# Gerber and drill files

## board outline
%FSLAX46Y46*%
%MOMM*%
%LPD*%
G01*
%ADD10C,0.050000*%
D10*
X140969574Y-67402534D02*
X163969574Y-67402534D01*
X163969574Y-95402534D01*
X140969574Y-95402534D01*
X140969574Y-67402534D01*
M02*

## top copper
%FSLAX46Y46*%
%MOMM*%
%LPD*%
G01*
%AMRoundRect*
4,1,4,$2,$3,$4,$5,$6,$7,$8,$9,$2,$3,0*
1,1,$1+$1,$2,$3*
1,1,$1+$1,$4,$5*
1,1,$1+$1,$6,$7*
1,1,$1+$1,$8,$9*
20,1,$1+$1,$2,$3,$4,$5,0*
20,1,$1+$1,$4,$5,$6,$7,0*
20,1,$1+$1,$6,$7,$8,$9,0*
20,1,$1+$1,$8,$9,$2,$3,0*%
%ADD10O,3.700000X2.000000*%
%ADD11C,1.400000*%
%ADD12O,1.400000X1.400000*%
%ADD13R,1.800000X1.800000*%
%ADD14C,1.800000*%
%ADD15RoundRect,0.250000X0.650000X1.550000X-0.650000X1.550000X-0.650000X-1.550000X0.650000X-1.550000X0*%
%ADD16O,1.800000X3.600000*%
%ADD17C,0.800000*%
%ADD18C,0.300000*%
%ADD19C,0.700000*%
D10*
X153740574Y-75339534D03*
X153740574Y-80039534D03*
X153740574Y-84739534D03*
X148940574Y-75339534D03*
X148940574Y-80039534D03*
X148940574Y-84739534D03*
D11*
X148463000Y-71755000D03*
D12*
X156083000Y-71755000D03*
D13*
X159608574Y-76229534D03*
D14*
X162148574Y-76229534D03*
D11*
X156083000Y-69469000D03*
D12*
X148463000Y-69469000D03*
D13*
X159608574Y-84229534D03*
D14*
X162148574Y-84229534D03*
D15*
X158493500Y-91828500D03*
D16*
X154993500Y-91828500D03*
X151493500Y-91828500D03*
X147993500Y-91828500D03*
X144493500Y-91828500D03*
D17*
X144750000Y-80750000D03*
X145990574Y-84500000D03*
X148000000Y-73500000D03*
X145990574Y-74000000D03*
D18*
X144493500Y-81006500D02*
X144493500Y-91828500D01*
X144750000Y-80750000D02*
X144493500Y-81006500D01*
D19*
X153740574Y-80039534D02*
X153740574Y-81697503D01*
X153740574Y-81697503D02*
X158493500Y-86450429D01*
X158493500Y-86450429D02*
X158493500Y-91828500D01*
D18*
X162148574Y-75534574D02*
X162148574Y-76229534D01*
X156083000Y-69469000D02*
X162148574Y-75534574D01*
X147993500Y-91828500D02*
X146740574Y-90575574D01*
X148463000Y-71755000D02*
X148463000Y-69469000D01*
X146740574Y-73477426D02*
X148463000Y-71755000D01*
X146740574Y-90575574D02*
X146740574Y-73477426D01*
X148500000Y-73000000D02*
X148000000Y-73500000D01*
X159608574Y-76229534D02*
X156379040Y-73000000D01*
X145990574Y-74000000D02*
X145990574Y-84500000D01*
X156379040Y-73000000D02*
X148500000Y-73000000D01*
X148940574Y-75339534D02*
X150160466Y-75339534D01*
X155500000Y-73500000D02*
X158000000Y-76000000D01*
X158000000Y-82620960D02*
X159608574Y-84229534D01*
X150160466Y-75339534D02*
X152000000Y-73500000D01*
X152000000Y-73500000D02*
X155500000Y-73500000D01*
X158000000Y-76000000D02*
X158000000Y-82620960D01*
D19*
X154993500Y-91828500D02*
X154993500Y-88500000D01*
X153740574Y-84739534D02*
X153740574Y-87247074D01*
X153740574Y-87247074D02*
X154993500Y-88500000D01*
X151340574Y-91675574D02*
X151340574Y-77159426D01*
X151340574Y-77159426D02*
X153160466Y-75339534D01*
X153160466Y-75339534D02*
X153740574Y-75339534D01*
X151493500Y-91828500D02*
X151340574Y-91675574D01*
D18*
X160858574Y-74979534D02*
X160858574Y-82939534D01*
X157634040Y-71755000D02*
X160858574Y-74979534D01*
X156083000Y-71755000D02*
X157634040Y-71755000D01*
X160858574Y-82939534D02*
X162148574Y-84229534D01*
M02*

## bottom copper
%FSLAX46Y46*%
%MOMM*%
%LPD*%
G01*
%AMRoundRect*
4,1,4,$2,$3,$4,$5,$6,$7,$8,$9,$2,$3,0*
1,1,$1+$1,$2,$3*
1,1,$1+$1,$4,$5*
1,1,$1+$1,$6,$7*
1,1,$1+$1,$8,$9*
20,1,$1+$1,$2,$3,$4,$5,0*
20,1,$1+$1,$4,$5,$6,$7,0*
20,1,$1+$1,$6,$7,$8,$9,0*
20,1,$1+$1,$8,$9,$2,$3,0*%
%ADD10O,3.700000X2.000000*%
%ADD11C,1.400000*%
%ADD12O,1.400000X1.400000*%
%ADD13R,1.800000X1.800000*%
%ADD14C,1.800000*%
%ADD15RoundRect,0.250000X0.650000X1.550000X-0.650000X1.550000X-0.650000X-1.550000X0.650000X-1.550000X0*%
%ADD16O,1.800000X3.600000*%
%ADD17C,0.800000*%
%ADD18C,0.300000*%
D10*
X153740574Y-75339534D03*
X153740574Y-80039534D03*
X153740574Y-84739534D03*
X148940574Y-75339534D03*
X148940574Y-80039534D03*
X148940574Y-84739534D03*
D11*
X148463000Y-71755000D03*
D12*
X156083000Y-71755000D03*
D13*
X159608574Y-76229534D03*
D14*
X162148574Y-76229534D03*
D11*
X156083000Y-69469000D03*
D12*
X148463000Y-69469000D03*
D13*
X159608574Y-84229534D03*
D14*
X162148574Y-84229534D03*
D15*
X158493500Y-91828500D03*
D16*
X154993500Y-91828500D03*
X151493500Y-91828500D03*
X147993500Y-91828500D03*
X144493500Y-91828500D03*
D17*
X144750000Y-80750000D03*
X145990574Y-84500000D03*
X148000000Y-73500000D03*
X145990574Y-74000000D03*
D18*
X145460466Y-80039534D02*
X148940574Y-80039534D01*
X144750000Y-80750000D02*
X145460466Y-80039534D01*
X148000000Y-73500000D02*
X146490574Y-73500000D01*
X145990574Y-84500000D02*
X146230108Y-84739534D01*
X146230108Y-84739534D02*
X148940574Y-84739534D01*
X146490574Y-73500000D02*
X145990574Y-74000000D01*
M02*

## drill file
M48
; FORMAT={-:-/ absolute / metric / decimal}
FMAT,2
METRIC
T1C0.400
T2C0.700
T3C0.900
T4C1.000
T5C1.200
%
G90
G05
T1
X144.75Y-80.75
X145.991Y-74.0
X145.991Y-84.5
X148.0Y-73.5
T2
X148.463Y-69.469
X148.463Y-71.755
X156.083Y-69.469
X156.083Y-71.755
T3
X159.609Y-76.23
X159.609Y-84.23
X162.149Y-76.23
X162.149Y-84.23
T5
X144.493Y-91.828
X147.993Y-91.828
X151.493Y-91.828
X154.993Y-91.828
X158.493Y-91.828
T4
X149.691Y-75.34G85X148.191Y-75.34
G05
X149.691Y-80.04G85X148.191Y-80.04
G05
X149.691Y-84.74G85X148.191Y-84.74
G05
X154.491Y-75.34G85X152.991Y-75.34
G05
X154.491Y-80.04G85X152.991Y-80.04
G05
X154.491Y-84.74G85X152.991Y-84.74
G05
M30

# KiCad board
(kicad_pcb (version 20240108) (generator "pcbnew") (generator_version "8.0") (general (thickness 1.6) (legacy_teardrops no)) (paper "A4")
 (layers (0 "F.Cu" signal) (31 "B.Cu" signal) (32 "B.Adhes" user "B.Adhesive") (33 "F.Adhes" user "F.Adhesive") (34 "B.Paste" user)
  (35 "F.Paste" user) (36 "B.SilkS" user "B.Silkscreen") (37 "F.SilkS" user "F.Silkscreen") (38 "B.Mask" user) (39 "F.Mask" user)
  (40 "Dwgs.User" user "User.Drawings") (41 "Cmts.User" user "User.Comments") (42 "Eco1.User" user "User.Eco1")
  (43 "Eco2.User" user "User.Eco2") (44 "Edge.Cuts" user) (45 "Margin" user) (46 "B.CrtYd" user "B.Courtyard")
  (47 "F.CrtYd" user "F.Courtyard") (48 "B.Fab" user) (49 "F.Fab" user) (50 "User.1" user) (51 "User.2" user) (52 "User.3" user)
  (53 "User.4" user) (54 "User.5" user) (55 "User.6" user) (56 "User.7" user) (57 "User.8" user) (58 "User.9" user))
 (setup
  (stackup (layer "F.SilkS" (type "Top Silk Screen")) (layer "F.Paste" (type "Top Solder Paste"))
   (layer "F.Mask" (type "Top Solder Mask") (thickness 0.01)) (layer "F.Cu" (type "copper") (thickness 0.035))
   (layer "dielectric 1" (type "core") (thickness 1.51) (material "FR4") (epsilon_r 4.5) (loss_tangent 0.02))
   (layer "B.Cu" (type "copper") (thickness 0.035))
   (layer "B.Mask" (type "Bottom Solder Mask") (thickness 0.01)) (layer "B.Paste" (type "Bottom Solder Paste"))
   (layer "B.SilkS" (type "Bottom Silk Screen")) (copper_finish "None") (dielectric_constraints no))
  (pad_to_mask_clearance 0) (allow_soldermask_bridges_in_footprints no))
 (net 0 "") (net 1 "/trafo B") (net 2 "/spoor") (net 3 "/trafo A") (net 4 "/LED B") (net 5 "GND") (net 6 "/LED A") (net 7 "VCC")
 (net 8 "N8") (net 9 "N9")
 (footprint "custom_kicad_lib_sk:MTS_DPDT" (layer "F.Cu") (at 150.740574 84.039534 -90)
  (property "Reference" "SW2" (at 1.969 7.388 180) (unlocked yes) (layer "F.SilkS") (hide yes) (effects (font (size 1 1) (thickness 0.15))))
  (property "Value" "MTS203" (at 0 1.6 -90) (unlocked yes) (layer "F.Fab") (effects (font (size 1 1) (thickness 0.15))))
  (pad "1" thru_hole oval (at -8.7 -3 270) (size 2 3.7) (drill oval 1 2.5) (layers "*.Cu" "*.Mask") (remove_unused_layers no)
   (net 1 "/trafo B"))
  (pad "2" thru_hole oval (at -4 -3 270) (size 2 3.7) (drill oval 1 2.5) (layers "*.Cu" "*.Mask") (remove_unused_layers no) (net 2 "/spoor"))
  (pad "3" thru_hole oval (at 0.7 -3 270) (size 2 3.7) (drill oval 1 2.5) (layers "*.Cu" "*.Mask") (remove_unused_layers no)
   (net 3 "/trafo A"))
  (pad "4" thru_hole oval (at -8.7 1.8 270) (size 2 3.7) (drill oval 1 2.5) (layers "*.Cu" "*.Mask") (remove_unused_layers no)
   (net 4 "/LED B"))
  (pad "5" thru_hole oval (at -4 1.8 270) (size 2 3.7) (drill oval 1 2.5) (layers "*.Cu" "*.Mask") (remove_unused_layers no) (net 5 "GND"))
  (pad "6" thru_hole oval (at 0.7 1.8 270) (size 2 3.7) (drill oval 1 2.5) (layers "*.Cu" "*.Mask") (remove_unused_layers no)
   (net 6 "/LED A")))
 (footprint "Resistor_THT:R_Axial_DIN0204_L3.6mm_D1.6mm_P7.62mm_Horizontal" (layer "F.Cu") (at 148.463 71.755)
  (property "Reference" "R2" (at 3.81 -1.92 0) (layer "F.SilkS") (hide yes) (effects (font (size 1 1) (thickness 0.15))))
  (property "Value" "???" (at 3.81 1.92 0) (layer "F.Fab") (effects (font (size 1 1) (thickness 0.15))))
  (pad "1" thru_hole circle (at 0 0) (size 1.4 1.4) (drill 0.7) (layers "*.Cu" "*.Mask") (remove_unused_layers no) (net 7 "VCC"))
  (pad "2" thru_hole oval (at 7.62 0) (size 1.4 1.4) (drill 0.7) (layers "*.Cu" "*.Mask") (remove_unused_layers no) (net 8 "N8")))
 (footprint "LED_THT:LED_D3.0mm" (layer "F.Cu") (at 159.608574 76.229534)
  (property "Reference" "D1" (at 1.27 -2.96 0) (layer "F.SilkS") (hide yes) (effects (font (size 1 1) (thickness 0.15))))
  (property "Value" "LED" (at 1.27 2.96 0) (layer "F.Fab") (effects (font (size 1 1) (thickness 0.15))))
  (pad "1" thru_hole rect (at 0 0) (size 1.8 1.8) (drill 0.9) (layers "*.Cu" "*.Mask") (remove_unused_layers no) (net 6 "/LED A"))
  (pad "2" thru_hole circle (at 2.54 0) (size 1.8 1.8) (drill 0.9) (layers "*.Cu" "*.Mask") (remove_unused_layers no) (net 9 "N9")))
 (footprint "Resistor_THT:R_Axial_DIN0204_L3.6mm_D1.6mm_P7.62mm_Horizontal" (layer "F.Cu") (at 156.083 69.469 180)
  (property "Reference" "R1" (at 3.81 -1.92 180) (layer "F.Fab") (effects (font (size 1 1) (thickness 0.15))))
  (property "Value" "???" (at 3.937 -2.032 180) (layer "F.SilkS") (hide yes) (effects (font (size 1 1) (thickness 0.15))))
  (pad "1" thru_hole circle (at 0 0 180) (size 1.4 1.4) (drill 0.7) (layers "*.Cu" "*.Mask") (remove_unused_layers no) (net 9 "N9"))
  (pad "2" thru_hole oval (at 7.62 0 180) (size 1.4 1.4) (drill 0.7) (layers "*.Cu" "*.Mask") (remove_unused_layers no) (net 7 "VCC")))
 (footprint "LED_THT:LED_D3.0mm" (layer "F.Cu") (at 159.608574 84.229534)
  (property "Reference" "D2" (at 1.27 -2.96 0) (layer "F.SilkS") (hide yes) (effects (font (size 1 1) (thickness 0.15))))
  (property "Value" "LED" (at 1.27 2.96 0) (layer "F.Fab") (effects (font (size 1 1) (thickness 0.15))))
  (pad "1" thru_hole rect (at 0 0) (size 1.8 1.8) (drill 0.9) (layers "*.Cu" "*.Mask") (remove_unused_layers no) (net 4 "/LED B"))
  (pad "2" thru_hole circle (at 2.54 0) (size 1.8 1.8) (drill 0.9) (layers "*.Cu" "*.Mask") (remove_unused_layers no) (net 8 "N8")))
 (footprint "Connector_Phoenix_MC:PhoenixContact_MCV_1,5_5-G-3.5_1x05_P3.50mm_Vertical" (layer "B.Cu") (at 158.4935 91.8285 180)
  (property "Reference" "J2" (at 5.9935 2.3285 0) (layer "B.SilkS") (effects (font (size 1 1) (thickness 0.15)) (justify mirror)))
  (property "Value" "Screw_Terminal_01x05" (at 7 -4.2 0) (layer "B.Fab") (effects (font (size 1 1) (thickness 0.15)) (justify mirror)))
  (pad "1" thru_hole roundrect (at 0 0 180) (size 1.8 3.6) (drill 1.2) (layers "*.Cu" "*.Mask") (remove_unused_layers no)
   (roundrect_rratio 0.138889) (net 2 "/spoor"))
  (pad "2" thru_hole oval (at 3.5 0 180) (size 1.8 3.6) (drill 1.2) (layers "*.Cu" "*.Mask") (remove_unused_layers no) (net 3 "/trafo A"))
  (pad "3" thru_hole oval (at 7 0 180) (size 1.8 3.6) (drill 1.2) (layers "*.Cu" "*.Mask") (remove_unused_layers no) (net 1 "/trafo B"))
  (pad "4" thru_hole oval (at 10.5 0 180) (size 1.8 3.6) (drill 1.2) (layers "*.Cu" "*.Mask") (remove_unused_layers no) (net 7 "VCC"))
  (pad "5" thru_hole oval (at 14 0 180) (size 1.8 3.6) (drill 1.2) (layers "*.Cu" "*.Mask") (remove_unused_layers no) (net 5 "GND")))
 (gr_rect (start 140.969574 67.402534) (end 163.969574 95.402534) (stroke (width 0.05) (type default)) (fill none) (layer "Edge.Cuts"))
 (segment (start 144.4935 81.0065) (end 144.4935 91.8285) (width 0.3) (layer "F.Cu") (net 5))
 (segment (start 144.75 80.75) (end 144.4935 81.0065) (width 0.3) (layer "F.Cu") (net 5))
 (via (at 144.75 80.75) (size 0.8) (drill 0.4) (layers "F.Cu" "B.Cu") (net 5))
 (segment (start 145.460466 80.039534) (end 148.940574 80.039534) (width 0.3) (layer "B.Cu") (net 5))
 (segment (start 144.75 80.75) (end 145.460466 80.039534) (width 0.3) (layer "B.Cu") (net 5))
 (segment (start 153.740574 80.039534) (end 153.740574 81.697503) (width 0.7) (layer "F.Cu") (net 2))
 (segment (start 153.740574 81.697503) (end 158.4935 86.450429) (width 0.7) (layer "F.Cu") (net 2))
 (segment (start 158.4935 86.450429) (end 158.4935 91.8285) (width 0.7) (layer "F.Cu") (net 2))
 (segment (start 162.148574 75.534574) (end 162.148574 76.229534) (width 0.3) (layer "F.Cu") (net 9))
 (segment (start 156.083 69.469) (end 162.148574 75.534574) (width 0.3) (layer "F.Cu") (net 9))
 (segment (start 147.9935 91.8285) (end 146.740574 90.575574) (width 0.3) (layer "F.Cu") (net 7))
 (segment (start 148.463 71.755) (end 148.463 69.469) (width 0.3) (layer "F.Cu") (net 7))
 (segment (start 146.740574 73.477426) (end 148.463 71.755) (width 0.3) (layer "F.Cu") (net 7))
 (segment (start 146.740574 90.575574) (end 146.740574 73.477426) (width 0.3) (layer "F.Cu") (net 7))
 (segment (start 148.5 73) (end 148 73.5) (width 0.3) (layer "F.Cu") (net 6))
 (segment (start 159.608574 76.229534) (end 156.37904 73) (width 0.3) (layer "F.Cu") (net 6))
 (segment (start 145.990574 74) (end 145.990574 84.5) (width 0.3) (layer "F.Cu") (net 6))
 (segment (start 156.37904 73) (end 148.5 73) (width 0.3) (layer "F.Cu") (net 6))
 (via (at 145.990574 84.5) (size 0.8) (drill 0.4) (layers "F.Cu" "B.Cu") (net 6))
 (via (at 148 73.5) (size 0.8) (drill 0.4) (layers "F.Cu" "B.Cu") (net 6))
 (via (at 145.990574 74) (size 0.8) (drill 0.4) (layers "F.Cu" "B.Cu") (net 6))
 (segment (start 148 73.5) (end 146.490574 73.5) (width 0.3) (layer "B.Cu") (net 6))
 (segment (start 145.990574 84.5) (end 146.230108 84.739534) (width 0.3) (layer "B.Cu") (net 6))
 (segment (start 146.230108 84.739534) (end 148.940574 84.739534) (width 0.3) (layer "B.Cu") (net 6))
 (segment (start 146.490574 73.5) (end 145.990574 74) (width 0.3) (layer "B.Cu") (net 6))
 (segment (start 148.940574 75.339534) (end 150.160466 75.339534) (width 0.3) (layer "F.Cu") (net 4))
 (segment (start 155.5 73.5) (end 158 76) (width 0.3) (layer "F.Cu") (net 4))
 (segment (start 158 82.62096) (end 159.608574 84.229534) (width 0.3) (layer "F.Cu") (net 4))
 (segment (start 150.160466 75.339534) (end 152 73.5) (width 0.3) (layer "F.Cu") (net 4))
 (segment (start 152 73.5) (end 155.5 73.5) (width 0.3) (layer "F.Cu") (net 4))
 (segment (start 158 76) (end 158 82.62096) (width 0.3) (layer "F.Cu") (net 4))
 (segment (start 154.9935 91.8285) (end 154.9935 88.5) (width 0.7) (layer "F.Cu") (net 3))
 (segment (start 153.740574 84.739534) (end 153.740574 87.247074) (width 0.7) (layer "F.Cu") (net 3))
 (segment (start 153.740574 87.247074) (end 154.9935 88.5) (width 0.7) (layer "F.Cu") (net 3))
 (segment (start 151.340574 91.675574) (end 151.340574 77.159426) (width 0.7) (layer "F.Cu") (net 1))
 (segment (start 151.340574 77.159426) (end 153.160466 75.339534) (width 0.7) (layer "F.Cu") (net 1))
 (segment (start 153.160466 75.339534) (end 153.740574 75.339534) (width 0.7) (layer "F.Cu") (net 1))
 (segment (start 151.4935 91.8285) (end 151.340574 91.675574) (width 0.7) (layer "F.Cu") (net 1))
 (segment (start 160.858574 74.979534) (end 160.858574 82.939534) (width 0.3) (layer "F.Cu") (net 8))
 (segment (start 157.63404 71.755) (end 160.858574 74.979534) (width 0.3) (layer "F.Cu") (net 8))
 (segment (start 156.083 71.755) (end 157.63404 71.755) (width 0.3) (layer "F.Cu") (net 8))
 (segment (start 160.858574 82.939534) (end 162.148574 84.229534) (width 0.3) (layer "F.Cu") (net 8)))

